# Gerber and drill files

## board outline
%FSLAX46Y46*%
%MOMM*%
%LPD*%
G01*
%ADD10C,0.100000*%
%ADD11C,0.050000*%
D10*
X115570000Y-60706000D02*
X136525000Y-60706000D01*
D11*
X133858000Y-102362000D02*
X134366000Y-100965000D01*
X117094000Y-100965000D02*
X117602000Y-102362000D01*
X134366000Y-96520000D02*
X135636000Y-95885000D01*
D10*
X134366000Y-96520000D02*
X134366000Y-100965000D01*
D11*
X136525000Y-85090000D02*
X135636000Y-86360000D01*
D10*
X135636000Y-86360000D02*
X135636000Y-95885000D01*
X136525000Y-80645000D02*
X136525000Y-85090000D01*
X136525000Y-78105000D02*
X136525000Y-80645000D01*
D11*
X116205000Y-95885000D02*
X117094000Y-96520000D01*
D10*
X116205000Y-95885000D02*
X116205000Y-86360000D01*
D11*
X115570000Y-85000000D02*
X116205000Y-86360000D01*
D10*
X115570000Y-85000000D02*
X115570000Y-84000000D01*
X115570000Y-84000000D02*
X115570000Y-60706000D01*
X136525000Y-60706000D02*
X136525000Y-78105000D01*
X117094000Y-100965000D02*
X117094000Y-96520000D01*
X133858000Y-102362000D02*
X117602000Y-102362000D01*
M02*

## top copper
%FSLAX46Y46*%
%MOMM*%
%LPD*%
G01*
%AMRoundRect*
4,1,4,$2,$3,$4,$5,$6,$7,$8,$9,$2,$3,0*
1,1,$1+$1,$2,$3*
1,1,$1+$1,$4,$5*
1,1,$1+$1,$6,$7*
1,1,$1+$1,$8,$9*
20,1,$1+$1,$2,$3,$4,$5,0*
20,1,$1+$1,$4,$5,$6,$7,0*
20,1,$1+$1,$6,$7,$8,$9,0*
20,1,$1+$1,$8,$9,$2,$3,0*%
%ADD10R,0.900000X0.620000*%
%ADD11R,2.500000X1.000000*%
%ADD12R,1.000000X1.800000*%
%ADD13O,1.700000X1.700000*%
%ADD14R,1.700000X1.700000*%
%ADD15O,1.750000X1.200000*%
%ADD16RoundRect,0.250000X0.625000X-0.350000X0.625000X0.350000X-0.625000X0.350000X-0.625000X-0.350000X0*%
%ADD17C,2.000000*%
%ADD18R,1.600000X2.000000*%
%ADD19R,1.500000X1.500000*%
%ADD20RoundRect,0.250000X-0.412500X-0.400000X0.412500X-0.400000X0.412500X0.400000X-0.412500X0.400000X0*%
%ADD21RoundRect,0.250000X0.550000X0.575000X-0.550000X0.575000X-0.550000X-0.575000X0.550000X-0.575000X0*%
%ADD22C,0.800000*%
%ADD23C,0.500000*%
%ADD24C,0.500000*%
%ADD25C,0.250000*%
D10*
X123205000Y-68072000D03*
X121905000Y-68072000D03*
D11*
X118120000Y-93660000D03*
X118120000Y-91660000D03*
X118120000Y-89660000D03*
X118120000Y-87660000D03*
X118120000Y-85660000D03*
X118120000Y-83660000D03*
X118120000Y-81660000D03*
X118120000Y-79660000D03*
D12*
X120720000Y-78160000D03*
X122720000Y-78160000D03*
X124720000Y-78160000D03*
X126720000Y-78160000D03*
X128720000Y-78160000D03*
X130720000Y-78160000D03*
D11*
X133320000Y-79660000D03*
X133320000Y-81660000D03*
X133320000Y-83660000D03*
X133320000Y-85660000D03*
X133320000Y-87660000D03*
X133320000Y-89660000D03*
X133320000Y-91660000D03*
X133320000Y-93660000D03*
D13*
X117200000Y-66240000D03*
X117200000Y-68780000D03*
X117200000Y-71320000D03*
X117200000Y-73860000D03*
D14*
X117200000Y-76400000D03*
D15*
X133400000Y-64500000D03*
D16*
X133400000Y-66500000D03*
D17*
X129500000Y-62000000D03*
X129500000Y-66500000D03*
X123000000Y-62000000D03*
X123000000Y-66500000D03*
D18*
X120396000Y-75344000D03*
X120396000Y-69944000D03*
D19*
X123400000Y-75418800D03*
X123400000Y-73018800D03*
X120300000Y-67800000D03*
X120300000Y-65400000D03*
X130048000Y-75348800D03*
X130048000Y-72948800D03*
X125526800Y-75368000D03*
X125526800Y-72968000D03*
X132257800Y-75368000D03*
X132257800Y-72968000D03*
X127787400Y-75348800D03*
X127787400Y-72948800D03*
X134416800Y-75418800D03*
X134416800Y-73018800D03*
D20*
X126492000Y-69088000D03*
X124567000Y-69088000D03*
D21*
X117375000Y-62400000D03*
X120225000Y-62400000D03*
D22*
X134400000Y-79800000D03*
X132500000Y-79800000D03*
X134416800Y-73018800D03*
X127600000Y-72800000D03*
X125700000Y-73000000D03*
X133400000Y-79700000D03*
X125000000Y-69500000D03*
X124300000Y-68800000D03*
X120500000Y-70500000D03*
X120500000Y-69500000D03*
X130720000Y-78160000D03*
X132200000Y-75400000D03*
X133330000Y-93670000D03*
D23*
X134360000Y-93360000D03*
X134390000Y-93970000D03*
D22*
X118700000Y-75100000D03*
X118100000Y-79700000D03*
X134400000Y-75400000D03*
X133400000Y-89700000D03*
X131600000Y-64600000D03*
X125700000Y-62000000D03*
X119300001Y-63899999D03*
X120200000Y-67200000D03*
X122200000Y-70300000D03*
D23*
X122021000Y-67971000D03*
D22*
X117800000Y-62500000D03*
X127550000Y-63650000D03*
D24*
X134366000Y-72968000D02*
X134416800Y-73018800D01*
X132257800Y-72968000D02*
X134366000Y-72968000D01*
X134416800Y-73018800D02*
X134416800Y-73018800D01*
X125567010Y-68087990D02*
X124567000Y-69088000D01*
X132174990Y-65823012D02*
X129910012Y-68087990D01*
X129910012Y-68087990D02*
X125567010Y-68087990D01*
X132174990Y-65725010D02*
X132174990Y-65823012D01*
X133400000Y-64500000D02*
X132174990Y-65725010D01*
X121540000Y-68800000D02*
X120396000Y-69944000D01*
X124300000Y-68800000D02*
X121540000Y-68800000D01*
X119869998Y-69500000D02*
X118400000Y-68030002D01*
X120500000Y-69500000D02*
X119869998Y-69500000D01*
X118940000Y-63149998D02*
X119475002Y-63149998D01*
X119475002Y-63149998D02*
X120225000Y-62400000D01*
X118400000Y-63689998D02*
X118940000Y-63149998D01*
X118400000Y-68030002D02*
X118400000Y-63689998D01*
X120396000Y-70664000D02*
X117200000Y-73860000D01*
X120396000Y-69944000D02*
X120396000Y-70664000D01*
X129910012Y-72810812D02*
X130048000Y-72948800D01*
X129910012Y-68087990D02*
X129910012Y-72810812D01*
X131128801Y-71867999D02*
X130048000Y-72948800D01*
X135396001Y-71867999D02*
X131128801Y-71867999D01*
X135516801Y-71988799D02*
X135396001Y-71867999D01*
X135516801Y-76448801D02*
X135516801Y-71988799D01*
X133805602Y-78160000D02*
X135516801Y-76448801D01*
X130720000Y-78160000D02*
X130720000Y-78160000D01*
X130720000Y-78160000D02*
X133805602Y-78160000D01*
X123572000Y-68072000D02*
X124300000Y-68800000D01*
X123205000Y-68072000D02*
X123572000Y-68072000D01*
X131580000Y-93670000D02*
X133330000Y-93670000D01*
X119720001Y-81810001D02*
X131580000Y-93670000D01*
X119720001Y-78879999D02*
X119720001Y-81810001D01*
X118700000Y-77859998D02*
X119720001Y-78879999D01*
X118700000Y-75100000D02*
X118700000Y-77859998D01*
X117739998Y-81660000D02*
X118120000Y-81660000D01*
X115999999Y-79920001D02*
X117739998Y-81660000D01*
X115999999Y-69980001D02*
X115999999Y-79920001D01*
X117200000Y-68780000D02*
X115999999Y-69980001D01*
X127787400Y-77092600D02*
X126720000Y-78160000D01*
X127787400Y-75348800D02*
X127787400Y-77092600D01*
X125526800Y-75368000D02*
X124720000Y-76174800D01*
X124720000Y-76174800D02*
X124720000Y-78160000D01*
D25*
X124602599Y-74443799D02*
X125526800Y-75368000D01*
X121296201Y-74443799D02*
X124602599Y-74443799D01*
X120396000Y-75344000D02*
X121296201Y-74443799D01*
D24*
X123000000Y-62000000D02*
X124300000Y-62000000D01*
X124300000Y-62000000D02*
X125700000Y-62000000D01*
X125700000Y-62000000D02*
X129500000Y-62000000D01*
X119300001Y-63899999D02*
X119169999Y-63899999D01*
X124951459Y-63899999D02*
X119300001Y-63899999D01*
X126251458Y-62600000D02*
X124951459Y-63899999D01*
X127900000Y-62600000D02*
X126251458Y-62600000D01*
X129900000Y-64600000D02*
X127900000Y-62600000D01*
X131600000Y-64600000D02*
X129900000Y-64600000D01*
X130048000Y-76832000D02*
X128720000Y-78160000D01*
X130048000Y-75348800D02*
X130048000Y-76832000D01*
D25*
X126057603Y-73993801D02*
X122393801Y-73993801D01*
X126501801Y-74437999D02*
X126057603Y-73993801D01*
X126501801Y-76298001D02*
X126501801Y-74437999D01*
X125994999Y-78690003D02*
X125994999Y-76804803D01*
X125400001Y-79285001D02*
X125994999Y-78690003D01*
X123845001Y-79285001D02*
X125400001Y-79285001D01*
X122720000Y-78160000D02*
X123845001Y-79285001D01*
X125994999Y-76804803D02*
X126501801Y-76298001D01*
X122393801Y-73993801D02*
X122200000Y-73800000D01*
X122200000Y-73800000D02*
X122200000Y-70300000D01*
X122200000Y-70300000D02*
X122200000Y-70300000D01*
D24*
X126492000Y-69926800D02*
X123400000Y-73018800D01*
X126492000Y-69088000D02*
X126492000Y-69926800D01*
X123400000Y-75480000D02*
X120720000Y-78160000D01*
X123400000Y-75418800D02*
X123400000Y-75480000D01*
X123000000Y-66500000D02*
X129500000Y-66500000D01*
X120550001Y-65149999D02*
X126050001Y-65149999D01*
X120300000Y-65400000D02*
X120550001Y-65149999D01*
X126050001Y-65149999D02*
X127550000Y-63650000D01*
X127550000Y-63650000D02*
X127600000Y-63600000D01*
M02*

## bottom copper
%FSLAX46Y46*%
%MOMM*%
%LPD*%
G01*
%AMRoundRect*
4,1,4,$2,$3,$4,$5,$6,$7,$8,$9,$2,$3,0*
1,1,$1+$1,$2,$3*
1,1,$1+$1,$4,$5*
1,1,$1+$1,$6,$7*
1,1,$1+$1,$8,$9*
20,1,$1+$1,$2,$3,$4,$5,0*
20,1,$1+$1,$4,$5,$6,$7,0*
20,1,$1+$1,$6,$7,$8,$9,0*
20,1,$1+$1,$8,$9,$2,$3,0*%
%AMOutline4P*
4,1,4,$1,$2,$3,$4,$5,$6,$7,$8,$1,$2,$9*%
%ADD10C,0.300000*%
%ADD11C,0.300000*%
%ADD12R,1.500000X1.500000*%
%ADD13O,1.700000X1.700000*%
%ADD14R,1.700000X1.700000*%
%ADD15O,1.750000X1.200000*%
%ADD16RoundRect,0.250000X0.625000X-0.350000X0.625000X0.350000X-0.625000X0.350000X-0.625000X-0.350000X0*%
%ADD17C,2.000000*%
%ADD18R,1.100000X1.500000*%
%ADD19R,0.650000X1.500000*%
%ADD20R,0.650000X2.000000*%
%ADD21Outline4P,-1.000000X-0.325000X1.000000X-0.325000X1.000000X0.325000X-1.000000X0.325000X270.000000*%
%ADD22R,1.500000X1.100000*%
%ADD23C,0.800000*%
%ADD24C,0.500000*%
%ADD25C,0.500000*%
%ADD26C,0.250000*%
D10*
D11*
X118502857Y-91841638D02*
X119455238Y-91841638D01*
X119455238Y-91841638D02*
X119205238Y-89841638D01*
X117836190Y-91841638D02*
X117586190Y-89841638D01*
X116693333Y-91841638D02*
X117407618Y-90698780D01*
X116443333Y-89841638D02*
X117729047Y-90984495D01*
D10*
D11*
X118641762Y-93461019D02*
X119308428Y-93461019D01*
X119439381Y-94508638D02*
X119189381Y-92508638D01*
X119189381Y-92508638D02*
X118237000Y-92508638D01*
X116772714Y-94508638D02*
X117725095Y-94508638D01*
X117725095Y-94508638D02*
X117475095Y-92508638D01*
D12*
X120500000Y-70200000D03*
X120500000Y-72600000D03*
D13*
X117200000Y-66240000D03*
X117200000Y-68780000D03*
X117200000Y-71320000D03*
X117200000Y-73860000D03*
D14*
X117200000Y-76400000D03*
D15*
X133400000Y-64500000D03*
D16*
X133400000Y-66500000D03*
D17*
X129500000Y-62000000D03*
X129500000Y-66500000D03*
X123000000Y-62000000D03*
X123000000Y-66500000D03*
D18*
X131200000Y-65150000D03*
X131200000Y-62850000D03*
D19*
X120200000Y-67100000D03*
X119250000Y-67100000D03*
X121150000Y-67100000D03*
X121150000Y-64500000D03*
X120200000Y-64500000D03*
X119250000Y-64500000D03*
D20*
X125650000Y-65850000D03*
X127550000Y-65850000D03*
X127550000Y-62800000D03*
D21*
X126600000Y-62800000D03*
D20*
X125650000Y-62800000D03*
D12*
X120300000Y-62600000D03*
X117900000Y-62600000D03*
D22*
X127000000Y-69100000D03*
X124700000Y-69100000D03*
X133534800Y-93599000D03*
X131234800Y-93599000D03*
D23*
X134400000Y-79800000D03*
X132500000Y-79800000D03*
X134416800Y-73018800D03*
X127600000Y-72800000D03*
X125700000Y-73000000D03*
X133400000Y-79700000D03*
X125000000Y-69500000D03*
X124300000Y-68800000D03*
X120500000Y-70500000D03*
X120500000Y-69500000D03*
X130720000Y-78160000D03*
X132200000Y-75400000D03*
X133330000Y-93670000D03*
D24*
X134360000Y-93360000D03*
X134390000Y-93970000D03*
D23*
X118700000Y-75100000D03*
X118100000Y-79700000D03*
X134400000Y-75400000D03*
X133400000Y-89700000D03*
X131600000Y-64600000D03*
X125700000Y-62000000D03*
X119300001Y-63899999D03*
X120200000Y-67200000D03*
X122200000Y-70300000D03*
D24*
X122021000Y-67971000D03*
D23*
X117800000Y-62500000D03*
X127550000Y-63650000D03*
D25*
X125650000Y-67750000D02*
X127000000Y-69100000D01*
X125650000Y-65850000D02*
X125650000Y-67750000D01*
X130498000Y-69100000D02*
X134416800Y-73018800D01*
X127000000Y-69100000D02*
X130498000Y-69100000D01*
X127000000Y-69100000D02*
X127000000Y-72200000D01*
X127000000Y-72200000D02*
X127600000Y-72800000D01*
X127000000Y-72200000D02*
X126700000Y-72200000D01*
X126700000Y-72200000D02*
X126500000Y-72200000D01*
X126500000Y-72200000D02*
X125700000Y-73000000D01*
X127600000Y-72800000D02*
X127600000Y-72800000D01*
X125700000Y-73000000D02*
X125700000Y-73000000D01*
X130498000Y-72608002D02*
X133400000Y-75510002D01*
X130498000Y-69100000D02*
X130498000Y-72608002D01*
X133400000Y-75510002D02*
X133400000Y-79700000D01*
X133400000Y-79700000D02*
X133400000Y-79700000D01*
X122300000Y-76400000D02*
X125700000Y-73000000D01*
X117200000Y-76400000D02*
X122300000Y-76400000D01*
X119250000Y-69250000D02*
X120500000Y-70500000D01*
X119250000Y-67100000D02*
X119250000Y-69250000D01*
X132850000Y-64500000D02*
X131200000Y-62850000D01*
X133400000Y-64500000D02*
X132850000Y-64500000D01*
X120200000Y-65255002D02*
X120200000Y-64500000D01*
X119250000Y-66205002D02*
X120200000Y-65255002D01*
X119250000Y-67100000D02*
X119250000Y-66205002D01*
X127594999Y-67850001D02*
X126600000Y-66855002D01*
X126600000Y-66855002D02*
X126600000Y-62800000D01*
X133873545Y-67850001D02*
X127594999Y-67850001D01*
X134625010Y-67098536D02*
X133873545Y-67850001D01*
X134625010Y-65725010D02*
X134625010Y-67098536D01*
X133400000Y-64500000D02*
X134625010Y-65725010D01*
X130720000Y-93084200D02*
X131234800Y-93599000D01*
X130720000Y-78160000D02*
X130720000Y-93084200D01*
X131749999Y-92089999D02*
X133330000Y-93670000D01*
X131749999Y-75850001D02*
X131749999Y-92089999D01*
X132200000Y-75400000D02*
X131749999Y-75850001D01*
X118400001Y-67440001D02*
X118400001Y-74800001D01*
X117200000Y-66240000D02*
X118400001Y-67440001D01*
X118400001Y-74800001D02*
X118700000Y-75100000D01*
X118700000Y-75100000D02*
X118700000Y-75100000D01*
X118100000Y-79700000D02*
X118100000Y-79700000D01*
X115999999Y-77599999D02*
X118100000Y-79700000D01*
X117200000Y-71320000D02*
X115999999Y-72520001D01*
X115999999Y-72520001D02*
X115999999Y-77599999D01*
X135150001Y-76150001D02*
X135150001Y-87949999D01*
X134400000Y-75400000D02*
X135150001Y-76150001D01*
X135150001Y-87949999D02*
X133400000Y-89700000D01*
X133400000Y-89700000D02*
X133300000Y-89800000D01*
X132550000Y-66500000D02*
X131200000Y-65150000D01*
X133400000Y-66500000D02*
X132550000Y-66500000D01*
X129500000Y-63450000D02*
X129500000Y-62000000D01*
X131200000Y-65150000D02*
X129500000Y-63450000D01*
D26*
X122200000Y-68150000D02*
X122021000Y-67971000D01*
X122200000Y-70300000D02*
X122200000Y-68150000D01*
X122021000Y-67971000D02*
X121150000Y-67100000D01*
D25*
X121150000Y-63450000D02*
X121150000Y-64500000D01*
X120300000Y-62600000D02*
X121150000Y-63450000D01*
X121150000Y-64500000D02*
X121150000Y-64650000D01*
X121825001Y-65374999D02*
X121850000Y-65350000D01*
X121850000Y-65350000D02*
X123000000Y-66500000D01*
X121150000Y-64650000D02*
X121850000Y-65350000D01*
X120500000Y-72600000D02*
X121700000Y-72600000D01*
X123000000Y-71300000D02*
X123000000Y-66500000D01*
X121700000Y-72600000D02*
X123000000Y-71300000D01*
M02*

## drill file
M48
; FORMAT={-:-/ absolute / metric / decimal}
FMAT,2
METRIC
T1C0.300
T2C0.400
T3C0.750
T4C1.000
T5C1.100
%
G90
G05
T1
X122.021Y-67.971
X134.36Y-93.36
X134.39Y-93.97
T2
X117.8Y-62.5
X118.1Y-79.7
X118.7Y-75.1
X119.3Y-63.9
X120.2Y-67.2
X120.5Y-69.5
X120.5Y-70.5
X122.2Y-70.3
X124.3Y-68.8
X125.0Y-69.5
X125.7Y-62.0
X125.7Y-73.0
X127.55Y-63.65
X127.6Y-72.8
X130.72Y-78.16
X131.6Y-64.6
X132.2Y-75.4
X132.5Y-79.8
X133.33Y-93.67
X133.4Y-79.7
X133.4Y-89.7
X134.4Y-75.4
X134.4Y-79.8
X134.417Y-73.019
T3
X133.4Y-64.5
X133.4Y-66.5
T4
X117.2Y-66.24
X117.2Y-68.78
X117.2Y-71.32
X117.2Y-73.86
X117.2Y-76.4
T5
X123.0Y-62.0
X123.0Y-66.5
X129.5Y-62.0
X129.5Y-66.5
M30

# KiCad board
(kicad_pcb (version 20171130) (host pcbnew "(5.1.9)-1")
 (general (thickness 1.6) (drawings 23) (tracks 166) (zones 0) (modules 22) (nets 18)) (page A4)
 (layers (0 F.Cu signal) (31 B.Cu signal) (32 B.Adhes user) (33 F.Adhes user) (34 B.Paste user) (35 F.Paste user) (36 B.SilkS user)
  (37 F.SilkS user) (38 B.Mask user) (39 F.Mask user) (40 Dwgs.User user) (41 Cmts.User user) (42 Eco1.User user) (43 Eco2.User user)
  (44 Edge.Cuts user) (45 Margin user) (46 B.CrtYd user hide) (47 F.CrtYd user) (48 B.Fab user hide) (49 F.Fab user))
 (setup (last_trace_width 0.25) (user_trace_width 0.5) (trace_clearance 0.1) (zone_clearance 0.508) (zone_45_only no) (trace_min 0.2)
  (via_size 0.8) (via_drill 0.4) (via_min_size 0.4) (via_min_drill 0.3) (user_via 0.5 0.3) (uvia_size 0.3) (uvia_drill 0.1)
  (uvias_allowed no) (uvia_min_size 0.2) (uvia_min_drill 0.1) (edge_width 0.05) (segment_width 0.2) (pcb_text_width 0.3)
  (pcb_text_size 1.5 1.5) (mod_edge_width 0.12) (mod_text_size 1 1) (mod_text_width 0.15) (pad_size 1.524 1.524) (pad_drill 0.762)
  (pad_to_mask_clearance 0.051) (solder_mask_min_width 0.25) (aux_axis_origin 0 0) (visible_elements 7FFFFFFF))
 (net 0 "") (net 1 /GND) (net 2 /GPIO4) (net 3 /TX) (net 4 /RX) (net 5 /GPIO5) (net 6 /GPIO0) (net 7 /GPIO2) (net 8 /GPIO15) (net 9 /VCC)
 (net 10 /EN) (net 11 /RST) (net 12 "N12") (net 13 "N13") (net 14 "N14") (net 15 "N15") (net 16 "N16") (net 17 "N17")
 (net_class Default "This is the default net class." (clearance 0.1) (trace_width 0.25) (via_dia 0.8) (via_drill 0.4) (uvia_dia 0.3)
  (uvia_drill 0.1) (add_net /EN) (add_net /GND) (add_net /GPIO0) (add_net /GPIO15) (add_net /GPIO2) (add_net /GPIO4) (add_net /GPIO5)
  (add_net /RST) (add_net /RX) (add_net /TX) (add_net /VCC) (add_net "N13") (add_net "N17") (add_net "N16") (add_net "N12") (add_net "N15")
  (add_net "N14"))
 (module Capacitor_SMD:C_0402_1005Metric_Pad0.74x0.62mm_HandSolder (layer F.Cu) (at 122.555 68.072)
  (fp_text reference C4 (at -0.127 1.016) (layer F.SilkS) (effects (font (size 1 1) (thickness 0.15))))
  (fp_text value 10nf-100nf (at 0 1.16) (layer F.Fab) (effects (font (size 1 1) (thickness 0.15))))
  (pad 2 smd rect (at 0.65 0) (size 0.9 0.62) (layers F.Cu F.Paste F.Mask) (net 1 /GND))
  (pad 1 smd rect (at -0.65 0) (size 0.9 0.62) (layers F.Cu F.Paste F.Mask) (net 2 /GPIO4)))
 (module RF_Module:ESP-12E (layer F.Cu) (at 125.72 90.16 180)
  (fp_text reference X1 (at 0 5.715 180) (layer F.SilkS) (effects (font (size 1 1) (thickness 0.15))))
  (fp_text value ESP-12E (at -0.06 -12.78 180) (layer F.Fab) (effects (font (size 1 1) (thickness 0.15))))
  (pad 22 smd rect (at 7.6 -3.5 180) (size 2.5 1) (layers F.Cu F.Paste F.Mask))
  (pad 21 smd rect (at 7.6 -1.5 180) (size 2.5 1) (layers F.Cu F.Paste F.Mask))
  (pad 20 smd rect (at 7.6 0.5 180) (size 2.5 1) (layers F.Cu F.Paste F.Mask))
  (pad 19 smd rect (at 7.6 2.5 180) (size 2.5 1) (layers F.Cu F.Paste F.Mask))
  (pad 18 smd rect (at 7.6 4.5 180) (size 2.5 1) (layers F.Cu F.Paste F.Mask))
  (pad 17 smd rect (at 7.6 6.5 180) (size 2.5 1) (layers F.Cu F.Paste F.Mask))
  (pad 16 smd rect (at 7.6 8.5 180) (size 2.5 1) (layers F.Cu F.Paste F.Mask) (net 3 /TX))
  (pad 15 smd rect (at 7.6 10.5 180) (size 2.5 1) (layers F.Cu F.Paste F.Mask) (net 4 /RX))
  (pad 14 smd rect (at 5 12 180) (size 1 1.8) (layers F.Cu F.Paste F.Mask) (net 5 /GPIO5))
  (pad 13 smd rect (at 3 12 180) (size 1 1.8) (layers F.Cu F.Paste F.Mask) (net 2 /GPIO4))
  (pad 12 smd rect (at 1 12 180) (size 1 1.8) (layers F.Cu F.Paste F.Mask) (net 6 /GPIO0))
  (pad 11 smd rect (at -1 12 180) (size 1 1.8) (layers F.Cu F.Paste F.Mask) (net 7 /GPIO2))
  (pad 10 smd rect (at -3 12 180) (size 1 1.8) (layers F.Cu F.Paste F.Mask) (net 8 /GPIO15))
  (pad 9 smd rect (at -5 12 180) (size 1 1.8) (layers F.Cu F.Paste F.Mask) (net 1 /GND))
  (pad 8 smd rect (at -7.6 10.5 180) (size 2.5 1) (layers F.Cu F.Paste F.Mask) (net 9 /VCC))
  (pad 7 smd rect (at -7.6 8.5 180) (size 2.5 1) (layers F.Cu F.Paste F.Mask))
  (pad 6 smd rect (at -7.6 6.5 180) (size 2.5 1) (layers F.Cu F.Paste F.Mask))
  (pad 5 smd rect (at -7.6 4.5 180) (size 2.5 1) (layers F.Cu F.Paste F.Mask))
  (pad 4 smd rect (at -7.6 2.5 180) (size 2.5 1) (layers F.Cu F.Paste F.Mask))
  (pad 3 smd rect (at -7.6 0.5 180) (size 2.5 1) (layers F.Cu F.Paste F.Mask) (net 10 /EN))
  (pad 2 smd rect (at -7.6 -1.5 180) (size 2.5 1) (layers F.Cu F.Paste F.Mask))
  (pad 1 smd rect (at -7.6 -3.5 180) (size 2.5 1) (layers F.Cu F.Paste F.Mask) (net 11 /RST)))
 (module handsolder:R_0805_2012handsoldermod (layer B.Cu) (at 120.5 71.4 90)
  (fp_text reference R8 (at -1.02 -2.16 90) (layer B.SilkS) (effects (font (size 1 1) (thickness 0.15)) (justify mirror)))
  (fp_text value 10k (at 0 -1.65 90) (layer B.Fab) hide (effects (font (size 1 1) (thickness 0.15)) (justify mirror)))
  (pad 2 smd rect (at 1.2 0 90) (size 1.5 1.5) (layers B.Cu B.Paste B.Mask) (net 1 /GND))
  (pad 1 smd rect (at -1.2 0 90) (size 1.5 1.5) (layers B.Cu B.Paste B.Mask) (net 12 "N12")))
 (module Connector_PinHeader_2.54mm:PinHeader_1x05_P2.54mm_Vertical (layer F.Cu) (at 117.2 76.4 180)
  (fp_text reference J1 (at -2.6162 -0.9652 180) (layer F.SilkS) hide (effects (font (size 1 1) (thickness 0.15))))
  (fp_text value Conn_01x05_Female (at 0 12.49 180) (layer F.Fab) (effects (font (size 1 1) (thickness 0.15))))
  (pad 5 thru_hole oval (at 0 10.16 180) (size 1.7 1.7) (drill 1) (layers *.Cu *.Mask) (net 11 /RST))
  (pad 4 thru_hole oval (at 0 7.62 180) (size 1.7 1.7) (drill 1) (layers *.Cu *.Mask) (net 3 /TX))
  (pad 3 thru_hole oval (at 0 5.08 180) (size 1.7 1.7) (drill 1) (layers *.Cu *.Mask) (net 4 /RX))
  (pad 2 thru_hole oval (at 0 2.54 180) (size 1.7 1.7) (drill 1) (layers *.Cu *.Mask) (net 1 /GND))
  (pad 1 thru_hole rect (at 0 0 180) (size 1.7 1.7) (drill 1) (layers *.Cu *.Mask) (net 9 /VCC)))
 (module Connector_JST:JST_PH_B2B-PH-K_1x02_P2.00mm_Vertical (layer F.Cu) (at 133.4 66.5 90)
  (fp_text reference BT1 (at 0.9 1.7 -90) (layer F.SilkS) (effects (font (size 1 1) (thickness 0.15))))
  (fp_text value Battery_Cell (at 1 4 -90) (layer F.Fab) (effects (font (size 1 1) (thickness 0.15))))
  (pad 2 thru_hole oval (at 2 0 90) (size 1.2 1.75) (drill 0.75) (layers *.Cu *.Mask) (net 1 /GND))
  (pad 1 thru_hole roundrect (at 0 0 90) (size 1.2 1.75) (drill 0.75) (layers *.Cu *.Mask) (roundrect_rratio 0.208333) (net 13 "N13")))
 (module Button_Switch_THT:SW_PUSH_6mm (layer F.Cu) (at 123 62)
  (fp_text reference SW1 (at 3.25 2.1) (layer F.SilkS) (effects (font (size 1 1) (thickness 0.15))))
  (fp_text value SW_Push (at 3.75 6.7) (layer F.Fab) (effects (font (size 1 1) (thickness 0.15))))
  (pad 1 thru_hole circle (at 6.5 0 90) (size 2 2) (drill 1.1) (layers *.Cu *.Mask) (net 13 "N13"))
  (pad 2 thru_hole circle (at 6.5 4.5 90) (size 2 2) (drill 1.1) (layers *.Cu *.Mask) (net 12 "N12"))
  (pad 1 thru_hole circle (at 0 0 90) (size 2 2) (drill 1.1) (layers *.Cu *.Mask) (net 13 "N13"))
  (pad 2 thru_hole circle (at 0 4.5 90) (size 2 2) (drill 1.1) (layers *.Cu *.Mask) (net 12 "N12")))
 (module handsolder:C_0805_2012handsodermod (layer B.Cu) (at 131.2 64 270)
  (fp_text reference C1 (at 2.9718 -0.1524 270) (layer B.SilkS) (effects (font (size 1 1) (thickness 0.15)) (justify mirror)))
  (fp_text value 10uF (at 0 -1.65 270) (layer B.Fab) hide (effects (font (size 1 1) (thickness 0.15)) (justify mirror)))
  (pad 2 smd rect (at 1.15 0 270) (size 1.5 1.1) (layers B.Cu B.Paste B.Mask) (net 13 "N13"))
  (pad 1 smd rect (at -1.15 0 270) (size 1.5 1.1) (layers B.Cu B.Paste B.Mask) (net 1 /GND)))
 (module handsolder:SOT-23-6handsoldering (layer B.Cu) (at 120.2 65.8 270)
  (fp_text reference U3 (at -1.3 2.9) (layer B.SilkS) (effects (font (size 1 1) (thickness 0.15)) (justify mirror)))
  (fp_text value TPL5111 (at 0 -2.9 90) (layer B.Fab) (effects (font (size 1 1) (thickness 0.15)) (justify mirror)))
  (pad 5 smd rect (at 1.3 0 270) (size 1.5 0.65) (layers B.Cu B.Paste B.Mask) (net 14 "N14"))
  (pad 6 smd rect (at 1.3 0.95 270) (size 1.5 0.65) (layers B.Cu B.Paste B.Mask) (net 1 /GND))
  (pad 4 smd rect (at 1.3 -0.95 270) (size 1.5 0.65) (layers B.Cu B.Paste B.Mask) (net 2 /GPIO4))
  (pad 3 smd rect (at -1.3 -0.95 270) (size 1.5 0.65) (layers B.Cu B.Paste B.Mask) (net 12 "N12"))
  (pad 2 smd rect (at -1.3 0 270) (size 1.5 0.65) (layers B.Cu B.Paste B.Mask) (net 1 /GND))
  (pad 1 smd rect (at -1.3 0.95 270) (size 1.5 0.65) (layers B.Cu B.Paste B.Mask) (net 13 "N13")))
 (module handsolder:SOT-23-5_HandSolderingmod (layer B.Cu) (at 126.6 64.35 270)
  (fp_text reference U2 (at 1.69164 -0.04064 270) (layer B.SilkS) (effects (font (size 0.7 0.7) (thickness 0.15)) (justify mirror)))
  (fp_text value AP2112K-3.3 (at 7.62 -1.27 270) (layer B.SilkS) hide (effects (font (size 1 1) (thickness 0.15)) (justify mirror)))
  (pad 5 smd rect (at 1.5 0.95 270) (size 2 0.65) (layers B.Cu B.Paste B.Mask) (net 9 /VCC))
  (pad 4 smd rect (at 1.5 -0.95 270) (size 2 0.65) (layers B.Cu B.Paste B.Mask))
  (pad 3 smd rect (at -1.55 -0.95 270) (size 2 0.65) (layers B.Cu B.Paste B.Mask) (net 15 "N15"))
  (pad 2 smd trapezoid (at -1.55 0 270) (size 2 0.65) (layers B.Cu B.Paste B.Mask) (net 1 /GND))
  (pad 1 smd rect (at -1.55 0.95 270) (size 2 0.65) (layers B.Cu B.Paste B.Mask) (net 13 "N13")))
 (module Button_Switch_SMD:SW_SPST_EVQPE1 (layer F.Cu) (at 120.396 72.644 90)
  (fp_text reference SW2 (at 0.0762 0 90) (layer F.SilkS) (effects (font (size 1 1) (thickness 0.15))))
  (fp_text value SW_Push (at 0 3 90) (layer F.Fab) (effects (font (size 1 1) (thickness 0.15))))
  (pad 1 smd rect (at -2.7 0 90) (size 2 1.6) (layers F.Cu F.Paste F.Mask) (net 6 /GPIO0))
  (pad 2 smd rect (at 2.7 0 90) (size 2 1.6) (layers F.Cu F.Paste F.Mask) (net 1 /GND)))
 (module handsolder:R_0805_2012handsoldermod (layer F.Cu) (at 123.4 74.2188 270)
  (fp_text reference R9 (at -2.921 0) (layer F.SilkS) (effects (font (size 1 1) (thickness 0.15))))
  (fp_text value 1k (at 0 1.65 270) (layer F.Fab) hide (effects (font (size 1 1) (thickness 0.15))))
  (pad 2 smd rect (at 1.2 0 270) (size 1.5 1.5) (layers F.Cu F.Paste F.Mask) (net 5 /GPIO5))
  (pad 1 smd rect (at -1.2 0 270) (size 1.5 1.5) (layers F.Cu F.Paste F.Mask) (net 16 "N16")))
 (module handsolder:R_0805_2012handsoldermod (layer F.Cu) (at 120.3 66.6 270)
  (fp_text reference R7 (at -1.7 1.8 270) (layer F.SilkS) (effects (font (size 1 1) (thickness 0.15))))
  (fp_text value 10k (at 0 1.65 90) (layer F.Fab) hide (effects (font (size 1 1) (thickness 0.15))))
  (pad 2 smd rect (at 1.2 0 270) (size 1.5 1.5) (layers F.Cu F.Paste F.Mask) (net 14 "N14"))
  (pad 1 smd rect (at -1.2 0 270) (size 1.5 1.5) (layers F.Cu F.Paste F.Mask) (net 15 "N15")))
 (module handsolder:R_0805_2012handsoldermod (layer B.Cu) (at 119.1 62.6)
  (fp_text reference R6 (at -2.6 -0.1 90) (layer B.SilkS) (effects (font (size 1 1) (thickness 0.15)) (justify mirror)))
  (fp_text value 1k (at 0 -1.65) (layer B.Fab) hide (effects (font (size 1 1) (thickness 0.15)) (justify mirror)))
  (pad 2 smd rect (at 1.2 0) (size 1.5 1.5) (layers B.Cu B.Paste B.Mask) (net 12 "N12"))
  (pad 1 smd rect (at -1.2 0) (size 1.5 1.5) (layers B.Cu B.Paste B.Mask) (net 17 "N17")))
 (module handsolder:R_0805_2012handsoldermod (layer F.Cu) (at 130.048 74.1488 270)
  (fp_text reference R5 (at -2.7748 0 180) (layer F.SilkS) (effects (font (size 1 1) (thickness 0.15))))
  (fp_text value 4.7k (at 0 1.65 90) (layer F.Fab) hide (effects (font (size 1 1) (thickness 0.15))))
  (pad 2 smd rect (at 1.2 0 270) (size 1.5 1.5) (layers F.Cu F.Paste F.Mask) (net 8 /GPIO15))
  (pad 1 smd rect (at -1.2 0 270) (size 1.5 1.5) (layers F.Cu F.Paste F.Mask) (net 1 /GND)))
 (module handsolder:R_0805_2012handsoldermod (layer F.Cu) (at 125.5268 74.168 270)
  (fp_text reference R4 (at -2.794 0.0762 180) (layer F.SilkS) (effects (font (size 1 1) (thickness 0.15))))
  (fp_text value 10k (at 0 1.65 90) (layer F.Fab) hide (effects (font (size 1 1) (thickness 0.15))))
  (pad 2 smd rect (at 1.2 0 270) (size 1.5 1.5) (layers F.Cu F.Paste F.Mask) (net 6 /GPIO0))
  (pad 1 smd rect (at -1.2 0 270) (size 1.5 1.5) (layers F.Cu F.Paste F.Mask) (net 9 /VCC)))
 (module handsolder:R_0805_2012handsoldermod (layer F.Cu) (at 132.2578 74.168 270)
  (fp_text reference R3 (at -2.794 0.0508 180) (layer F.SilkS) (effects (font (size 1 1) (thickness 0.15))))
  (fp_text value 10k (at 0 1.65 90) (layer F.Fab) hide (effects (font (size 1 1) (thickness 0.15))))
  (pad 2 smd rect (at 1.2 0 270) (size 1.5 1.5) (layers F.Cu F.Paste F.Mask) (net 11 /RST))
  (pad 1 smd rect (at -1.2 0 270) (size 1.5 1.5) (layers F.Cu F.Paste F.Mask) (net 9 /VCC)))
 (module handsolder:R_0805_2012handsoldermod (layer F.Cu) (at 127.7874 74.1488 270)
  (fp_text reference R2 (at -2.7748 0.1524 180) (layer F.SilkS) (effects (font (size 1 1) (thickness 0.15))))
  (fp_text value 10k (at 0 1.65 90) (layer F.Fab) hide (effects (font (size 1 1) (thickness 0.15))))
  (pad 2 smd rect (at 1.2 0 270) (size 1.5 1.5) (layers F.Cu F.Paste F.Mask) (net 7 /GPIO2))
  (pad 1 smd rect (at -1.2 0 270) (size 1.5 1.5) (layers F.Cu F.Paste F.Mask) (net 9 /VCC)))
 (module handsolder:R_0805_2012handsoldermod (layer F.Cu) (at 134.4168 74.2188 270)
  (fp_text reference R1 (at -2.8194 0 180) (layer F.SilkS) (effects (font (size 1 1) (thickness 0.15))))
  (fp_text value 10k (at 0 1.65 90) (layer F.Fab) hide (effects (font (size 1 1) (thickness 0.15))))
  (pad 2 smd rect (at 1.2 0 270) (size 1.5 1.5) (layers F.Cu F.Paste F.Mask) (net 10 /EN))
  (pad 1 smd rect (at -1.2 0 270) (size 1.5 1.5) (layers F.Cu F.Paste F.Mask) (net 9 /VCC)))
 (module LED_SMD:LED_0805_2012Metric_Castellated (layer F.Cu) (at 125.5295 69.088)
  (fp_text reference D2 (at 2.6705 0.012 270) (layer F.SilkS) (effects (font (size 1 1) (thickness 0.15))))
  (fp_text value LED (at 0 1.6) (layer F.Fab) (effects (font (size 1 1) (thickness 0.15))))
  (pad 2 smd roundrect (at 0.9625 0) (size 1.325 1.3) (layers F.Cu F.Paste F.Mask) (roundrect_rratio 0.1923076923076923) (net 16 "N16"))
  (pad 1 smd roundrect (at -0.9625 0) (size 1.325 1.3) (layers F.Cu F.Paste F.Mask) (roundrect_rratio 0.1923076923076923) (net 1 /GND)))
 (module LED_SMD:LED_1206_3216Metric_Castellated (layer F.Cu) (at 118.8 62.4 180)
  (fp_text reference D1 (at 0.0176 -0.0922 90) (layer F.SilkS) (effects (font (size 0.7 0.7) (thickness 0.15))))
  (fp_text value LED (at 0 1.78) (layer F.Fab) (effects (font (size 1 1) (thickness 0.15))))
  (pad 2 smd roundrect (at 1.425 0 180) (size 1.6 1.65) (layers F.Cu F.Paste F.Mask) (roundrect_rratio 0.15625) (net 17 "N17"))
  (pad 1 smd roundrect (at -1.425 0 180) (size 1.6 1.65) (layers F.Cu F.Paste F.Mask) (roundrect_rratio 0.15625) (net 1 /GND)))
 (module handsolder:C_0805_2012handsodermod (layer B.Cu) (at 125.85 69.1)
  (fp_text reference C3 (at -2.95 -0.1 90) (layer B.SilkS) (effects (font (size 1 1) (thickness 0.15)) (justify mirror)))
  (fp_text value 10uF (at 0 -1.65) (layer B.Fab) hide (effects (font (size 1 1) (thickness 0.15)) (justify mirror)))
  (pad 2 smd rect (at 1.15 0) (size 1.5 1.1) (layers B.Cu B.Paste B.Mask) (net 9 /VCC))
  (pad 1 smd rect (at -1.15 0) (size 1.5 1.1) (layers B.Cu B.Paste B.Mask) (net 1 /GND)))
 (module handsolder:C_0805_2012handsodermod (layer B.Cu) (at 132.3848 93.599)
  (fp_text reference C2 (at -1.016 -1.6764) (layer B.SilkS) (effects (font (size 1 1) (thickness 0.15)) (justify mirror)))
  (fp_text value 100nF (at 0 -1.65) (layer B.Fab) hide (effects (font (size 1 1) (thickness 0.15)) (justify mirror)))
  (pad 2 smd rect (at 1.15 0) (size 1.5 1.1) (layers B.Cu B.Paste B.Mask) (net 11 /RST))
  (pad 1 smd rect (at -1.15 0) (size 1.5 1.1) (layers B.Cu B.Paste B.Mask) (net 1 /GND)))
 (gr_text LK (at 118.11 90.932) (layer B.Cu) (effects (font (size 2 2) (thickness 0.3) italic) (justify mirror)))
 (gr_line (start 115.57 60.706) (end 136.525 60.706) (layer Edge.Cuts) (width 0.1))
 (gr_line (start 133.858 102.362) (end 134.366 100.965) (layer Edge.Cuts) (width 0.05))
 (gr_line (start 117.094 100.965) (end 117.602 102.362) (layer Edge.Cuts) (width 0.05))
 (gr_line (start 134.366 96.52) (end 135.636 95.885) (layer Edge.Cuts) (width 0.05))
 (gr_line (start 134.366 96.52) (end 134.366 100.965) (layer Edge.Cuts) (width 0.1))
 (gr_line (start 136.525 85.09) (end 135.636 86.36) (layer Edge.Cuts) (width 0.05))
 (gr_line (start 135.636 86.36) (end 135.636 95.885) (layer Edge.Cuts) (width 0.1))
 (gr_line (start 136.525 80.645) (end 136.525 85.09) (layer Edge.Cuts) (width 0.1))
 (gr_line (start 136.525 78.105) (end 136.525 80.645) (layer Edge.Cuts) (width 0.1))
 (gr_line (start 116.205 95.885) (end 117.094 96.52) (layer Edge.Cuts) (width 0.05))
 (gr_line (start 116.205 95.885) (end 116.205 86.36) (layer Edge.Cuts) (width 0.1))
 (gr_line (start 115.57 85) (end 116.205 86.36) (layer Edge.Cuts) (width 0.05))
 (gr_line (start 115.57 85) (end 115.57 84) (layer Edge.Cuts) (width 0.1))
 (gr_line (start 115.57 84) (end 115.57 60.706) (layer Edge.Cuts) (width 0.1))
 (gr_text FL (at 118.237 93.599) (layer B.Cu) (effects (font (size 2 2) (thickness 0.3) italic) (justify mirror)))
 (gr_line (start 136.525 60.706) (end 136.525 78.105) (layer Edge.Cuts) (width 0.1))
 (gr_line (start 117.094 100.965) (end 117.094 96.52) (layer Edge.Cuts) (width 0.1))
 (gr_line (start 133.858 102.362) (end 117.602 102.362) (layer Edge.Cuts) (width 0.1))
 (via (at 134.4 79.8) (size 0.8) (drill 0.4) (layers F.Cu B.Cu) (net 9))
 (via (at 132.5 79.8) (size 0.8) (drill 0.4) (layers F.Cu B.Cu) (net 9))
 (segment (start 125.65 67.75) (end 127 69.1) (width 0.5) (layer B.Cu) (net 9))
 (segment (start 125.65 65.85) (end 125.65 67.75) (width 0.5) (layer B.Cu) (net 9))
 (segment (start 134.366 72.968) (end 134.4168 73.0188) (width 0.5) (layer F.Cu) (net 9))
 (segment (start 132.2578 72.968) (end 134.366 72.968) (width 0.5) (layer F.Cu) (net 9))
 (segment (start 134.4168 73.0188) (end 134.4168 73.0188) (width 0.5) (layer F.Cu) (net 9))
 (via (at 134.4168 73.0188) (size 0.8) (drill 0.4) (layers F.Cu B.Cu) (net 9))
 (segment (start 130.498 69.1) (end 134.4168 73.0188) (width 0.5) (layer B.Cu) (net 9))
 (segment (start 127 69.1) (end 130.498 69.1) (width 0.5) (layer B.Cu) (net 9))
 (segment (start 127 69.1) (end 127 72.2) (width 0.5) (layer B.Cu) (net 9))
 (segment (start 127 72.2) (end 127.6 72.8) (width 0.5) (layer B.Cu) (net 9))
 (segment (start 127 72.2) (end 126.7 72.2) (width 0.5) (layer B.Cu) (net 9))
 (segment (start 126.7 72.2) (end 126.5 72.2) (width 0.5) (layer B.Cu) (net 9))
 (segment (start 126.5 72.2) (end 125.7 73) (width 0.5) (layer B.Cu) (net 9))
 (segment (start 127.6 72.8) (end 127.6 72.8) (width 0.5) (layer B.Cu) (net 9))
 (via (at 127.6 72.8) (size 0.8) (drill 0.4) (layers F.Cu B.Cu) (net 9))
 (segment (start 125.7 73) (end 125.7 73) (width 0.5) (layer B.Cu) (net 9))
 (via (at 125.7 73) (size 0.8) (drill 0.4) (layers F.Cu B.Cu) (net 9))
 (segment (start 130.498 72.608002) (end 133.4 75.510002) (width 0.5) (layer B.Cu) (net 9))
 (segment (start 130.498 69.1) (end 130.498 72.608002) (width 0.5) (layer B.Cu) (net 9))
 (segment (start 133.4 75.510002) (end 133.4 79.7) (width 0.5) (layer B.Cu) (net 9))
 (segment (start 133.4 79.7) (end 133.4 79.7) (width 0.5) (layer B.Cu) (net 9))
 (via (at 133.4 79.7) (size 0.8) (drill 0.4) (layers F.Cu B.Cu) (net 9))
 (segment (start 122.3 76.4) (end 125.7 73) (width 0.5) (layer B.Cu) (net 9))
 (segment (start 117.2 76.4) (end 122.3 76.4) (width 0.5) (layer B.Cu) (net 9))
 (via (at 125 69.5) (size 0.8) (drill 0.4) (layers F.Cu B.Cu) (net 1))
 (via (at 124.3 68.8) (size 0.8) (drill 0.4) (layers F.Cu B.Cu) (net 1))
 (via (at 120.5 70.5) (size 0.8) (drill 0.4) (layers F.Cu B.Cu) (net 1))
 (via (at 120.5 69.5) (size 0.8) (drill 0.4) (layers F.Cu B.Cu) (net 1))
 (segment (start 119.25 69.25) (end 120.5 70.5) (width 0.5) (layer B.Cu) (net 1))
 (segment (start 119.25 67.1) (end 119.25 69.25) (width 0.5) (layer B.Cu) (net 1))
 (segment (start 132.85 64.5) (end 131.2 62.85) (width 0.5) (layer B.Cu) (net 1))
 (segment (start 133.4 64.5) (end 132.85 64.5) (width 0.5) (layer B.Cu) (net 1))
 (segment (start 120.2 65.255002) (end 120.2 64.5) (width 0.5) (layer B.Cu) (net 1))
 (segment (start 119.25 66.205002) (end 120.2 65.255002) (width 0.5) (layer B.Cu) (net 1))
 (segment (start 119.25 67.1) (end 119.25 66.205002) (width 0.5) (layer B.Cu) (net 1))
 (segment (start 127.594999 67.850001) (end 126.6 66.855002) (width 0.5) (layer B.Cu) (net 1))
 (segment (start 126.6 66.855002) (end 126.6 62.8) (width 0.5) (layer B.Cu) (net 1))
 (segment (start 133.873545 67.850001) (end 127.594999 67.850001) (width 0.5) (layer B.Cu) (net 1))
 (segment (start 134.62501 67.098536) (end 133.873545 67.850001) (width 0.5) (layer B.Cu) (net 1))
 (segment (start 134.62501 65.72501) (end 134.62501 67.098536) (width 0.5) (layer B.Cu) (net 1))
 (segment (start 133.4 64.5) (end 134.62501 65.72501) (width 0.5) (layer B.Cu) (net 1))
 (segment (start 125.56701 68.08799) (end 124.567 69.088) (width 0.5) (layer F.Cu) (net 1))
 (segment (start 132.17499 65.823012) (end 129.910012 68.08799) (width 0.5) (layer F.Cu) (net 1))
 (segment (start 129.910012 68.08799) (end 125.56701 68.08799) (width 0.5) (layer F.Cu) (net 1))
 (segment (start 132.17499 65.72501) (end 132.17499 65.823012) (width 0.5) (layer F.Cu) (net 1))
 (segment (start 133.4 64.5) (end 132.17499 65.72501) (width 0.5) (layer F.Cu) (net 1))
 (segment (start 121.54 68.8) (end 120.396 69.944) (width 0.5) (layer F.Cu) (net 1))
 (segment (start 124.3 68.8) (end 121.54 68.8) (width 0.5) (layer F.Cu) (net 1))
 (segment (start 119.869998 69.5) (end 118.4 68.030002) (width 0.5) (layer F.Cu) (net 1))
 (segment (start 120.5 69.5) (end 119.869998 69.5) (width 0.5) (layer F.Cu) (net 1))
 (segment (start 118.94 63.149998) (end 119.475002 63.149998) (width 0.5) (layer F.Cu) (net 1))
 (segment (start 119.475002 63.149998) (end 120.225 62.4) (width 0.5) (layer F.Cu) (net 1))
 (segment (start 118.4 63.689998) (end 118.94 63.149998) (width 0.5) (layer F.Cu) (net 1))
 (segment (start 118.4 68.030002) (end 118.4 63.689998) (width 0.5) (layer F.Cu) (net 1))
 (segment (start 120.396 70.664) (end 117.2 73.86) (width 0.5) (layer F.Cu) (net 1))
 (segment (start 120.396 69.944) (end 120.396 70.664) (width 0.5) (layer F.Cu) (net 1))
 (segment (start 129.910012 72.810812) (end 130.048 72.9488) (width 0.5) (layer F.Cu) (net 1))
 (segment (start 129.910012 68.08799) (end 129.910012 72.810812) (width 0.5) (layer F.Cu) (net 1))
 (segment (start 131.128801 71.867999) (end 130.048 72.9488) (width 0.5) (layer F.Cu) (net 1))
 (segment (start 135.396001 71.867999) (end 131.128801 71.867999) (width 0.5) (layer F.Cu) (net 1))
 (segment (start 135.516801 71.988799) (end 135.396001 71.867999) (width 0.5) (layer F.Cu) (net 1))
 (segment (start 135.516801 76.448801) (end 135.516801 71.988799) (width 0.5) (layer F.Cu) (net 1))
 (segment (start 133.805602 78.16) (end 135.516801 76.448801) (width 0.5) (layer F.Cu) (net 1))
 (segment (start 130.72 78.16) (end 130.72 78.16) (width 0.5) (layer F.Cu) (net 1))
 (segment (start 130.72 78.16) (end 133.805602 78.16) (width 0.5) (layer F.Cu) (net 1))
 (via (at 130.72 78.16) (size 0.8) (drill 0.4) (layers F.Cu B.Cu) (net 1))
 (segment (start 130.72 93.0842) (end 131.2348 93.599) (width 0.5) (layer B.Cu) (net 1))
 (segment (start 130.72 78.16) (end 130.72 93.0842) (width 0.5) (layer B.Cu) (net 1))
 (segment (start 123.572 68.072) (end 124.3 68.8) (width 0.5) (layer F.Cu) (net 1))
 (segment (start 123.205 68.072) (end 123.572 68.072) (width 0.5) (layer F.Cu) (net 1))
 (via (at 132.2 75.4) (size 0.8) (drill 0.4) (layers F.Cu B.Cu) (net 11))
 (via (at 133.33 93.67) (size 0.8) (drill 0.4) (layers F.Cu B.Cu) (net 11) (status 30))
 (via (at 134.36 93.36) (size 0.5) (drill 0.3) (layers F.Cu B.Cu) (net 11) (status 30))
 (via (at 134.39 93.97) (size 0.5) (drill 0.3) (layers F.Cu B.Cu) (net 11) (status 30))
 (segment (start 131.749999 92.089999) (end 133.33 93.67) (width 0.5) (layer B.Cu) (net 11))
 (segment (start 131.749999 75.850001) (end 131.749999 92.089999) (width 0.5) (layer B.Cu) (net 11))
 (segment (start 132.2 75.4) (end 131.749999 75.850001) (width 0.5) (layer B.Cu) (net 11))
 (segment (start 118.400001 67.440001) (end 118.400001 74.800001) (width 0.5) (layer B.Cu) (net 11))
 (segment (start 117.2 66.24) (end 118.400001 67.440001) (width 0.5) (layer B.Cu) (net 11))
 (segment (start 118.400001 74.800001) (end 118.7 75.1) (width 0.5) (layer B.Cu) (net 11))
 (segment (start 118.7 75.1) (end 118.7 75.1) (width 0.5) (layer B.Cu) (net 11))
 (via (at 118.7 75.1) (size 0.8) (drill 0.4) (layers F.Cu B.Cu) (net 11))
 (segment (start 131.58 93.67) (end 133.33 93.67) (width 0.5) (layer F.Cu) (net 11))
 (segment (start 119.720001 81.810001) (end 131.58 93.67) (width 0.5) (layer F.Cu) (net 11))
 (segment (start 119.720001 78.879999) (end 119.720001 81.810001) (width 0.5) (layer F.Cu) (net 11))
 (segment (start 118.7 77.859998) (end 119.720001 78.879999) (width 0.5) (layer F.Cu) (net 11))
 (segment (start 118.7 75.1) (end 118.7 77.859998) (width 0.5) (layer F.Cu) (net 11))
 (segment (start 118.1 79.7) (end 118.1 79.7) (width 0.5) (layer B.Cu) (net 4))
 (via (at 118.1 79.7) (size 0.8) (drill 0.4) (layers F.Cu B.Cu) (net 4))
 (segment (start 115.999999 77.599999) (end 118.1 79.7) (width 0.5) (layer B.Cu) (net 4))
 (segment (start 117.2 71.32) (end 115.999999 72.520001) (width 0.5) (layer B.Cu) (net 4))
 (segment (start 115.999999 72.520001) (end 115.999999 77.599999) (width 0.5) (layer B.Cu) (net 4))
 (segment (start 117.739998 81.66) (end 118.12 81.66) (width 0.5) (layer F.Cu) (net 3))
 (segment (start 115.999999 79.920001) (end 117.739998 81.66) (width 0.5) (layer F.Cu) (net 3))
 (segment (start 115.999999 69.980001) (end 115.999999 79.920001) (width 0.5) (layer F.Cu) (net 3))
 (segment (start 117.2 68.78) (end 115.999999 69.980001) (width 0.5) (layer F.Cu) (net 3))
 (via (at 134.4 75.4) (size 0.8) (drill 0.4) (layers F.Cu B.Cu) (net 10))
 (segment (start 135.150001 76.150001) (end 135.150001 87.949999) (width 0.5) (layer B.Cu) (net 10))
 (segment (start 134.4 75.4) (end 135.150001 76.150001) (width 0.5) (layer B.Cu) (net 10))
 (segment (start 135.150001 87.949999) (end 133.4 89.7) (width 0.5) (layer B.Cu) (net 10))
 (segment (start 133.4 89.7) (end 133.3 89.8) (width 0.5) (layer B.Cu) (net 10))
 (via (at 133.4 89.7) (size 0.8) (drill 0.4) (layers F.Cu B.Cu) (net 10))
 (segment (start 127.7874 77.0926) (end 126.72 78.16) (width 0.5) (layer F.Cu) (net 7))
 (segment (start 127.7874 75.3488) (end 127.7874 77.0926) (width 0.5) (layer F.Cu) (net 7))
 (segment (start 125.5268 75.368) (end 124.72 76.1748) (width 0.5) (layer F.Cu) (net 6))
 (segment (start 124.72 76.1748) (end 124.72 78.16) (width 0.5) (layer F.Cu) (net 6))
 (segment (start 124.602599 74.443799) (end 125.5268 75.368) (width 0.25) (layer F.Cu) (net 6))
 (segment (start 121.296201 74.443799) (end 124.602599 74.443799) (width 0.25) (layer F.Cu) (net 6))
 (segment (start 120.396 75.344) (end 121.296201 74.443799) (width 0.25) (layer F.Cu) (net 6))
 (via (at 131.6 64.6) (size 0.8) (drill 0.4) (layers F.Cu B.Cu) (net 13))
 (segment (start 123 62) (end 124.3 62) (width 0.5) (layer F.Cu) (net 13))
 (segment (start 124.3 62) (end 125.7 62) (width 0.5) (layer F.Cu) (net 13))
 (segment (start 125.7 62) (end 129.5 62) (width 0.5) (layer F.Cu) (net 13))
 (via (at 125.7 62) (size 0.8) (drill 0.4) (layers F.Cu B.Cu) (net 13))
 (segment (start 132.55 66.5) (end 131.2 65.15) (width 0.5) (layer B.Cu) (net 13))
 (segment (start 133.4 66.5) (end 132.55 66.5) (width 0.5) (layer B.Cu) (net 13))
 (segment (start 129.5 63.45) (end 129.5 62) (width 0.5) (layer B.Cu) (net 13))
 (segment (start 131.2 65.15) (end 129.5 63.45) (width 0.5) (layer B.Cu) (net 13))
 (segment (start 119.300001 63.899999) (end 119.169999 63.899999) (width 0.5) (layer F.Cu) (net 13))
 (via (at 119.300001 63.899999) (size 0.8) (drill 0.4) (layers F.Cu B.Cu) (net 13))
 (segment (start 124.951459 63.899999) (end 119.300001 63.899999) (width 0.5) (layer F.Cu) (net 13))
 (segment (start 126.251458 62.6) (end 124.951459 63.899999) (width 0.5) (layer F.Cu) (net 13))
 (segment (start 127.9 62.6) (end 126.251458 62.6) (width 0.5) (layer F.Cu) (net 13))
 (segment (start 129.9 64.6) (end 127.9 62.6) (width 0.5) (layer F.Cu) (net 13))
 (segment (start 131.6 64.6) (end 129.9 64.6) (width 0.5) (layer F.Cu) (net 13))
 (segment (start 130.048 76.832) (end 128.72 78.16) (width 0.5) (layer F.Cu) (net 8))
 (segment (start 130.048 75.3488) (end 130.048 76.832) (width 0.5) (layer F.Cu) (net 8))
 (via (at 120.2 67.2) (size 0.8) (drill 0.4) (layers F.Cu B.Cu) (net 14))
 (segment (start 126.057603 73.993801) (end 122.393801 73.993801) (width 0.25) (layer F.Cu) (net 2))
 (segment (start 126.501801 74.437999) (end 126.057603 73.993801) (width 0.25) (layer F.Cu) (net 2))
 (segment (start 126.501801 76.298001) (end 126.501801 74.437999) (width 0.25) (layer F.Cu) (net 2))
 (segment (start 125.994999 78.690003) (end 125.994999 76.804803) (width 0.25) (layer F.Cu) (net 2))
 (segment (start 125.400001 79.285001) (end 125.994999 78.690003) (width 0.25) (layer F.Cu) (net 2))
 (segment (start 123.845001 79.285001) (end 125.400001 79.285001) (width 0.25) (layer F.Cu) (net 2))
 (segment (start 122.72 78.16) (end 123.845001 79.285001) (width 0.25) (layer F.Cu) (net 2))
 (segment (start 125.994999 76.804803) (end 126.501801 76.298001) (width 0.25) (layer F.Cu) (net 2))
 (segment (start 122.393801 73.993801) (end 122.2 73.8) (width 0.25) (layer F.Cu) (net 2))
 (segment (start 122.2 73.8) (end 122.2 70.3) (width 0.25) (layer F.Cu) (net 2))
 (segment (start 122.2 70.3) (end 122.2 70.3) (width 0.25) (layer F.Cu) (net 2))
 (via (at 122.2 70.3) (size 0.8) (drill 0.4) (layers F.Cu B.Cu) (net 2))
 (segment (start 122.2 68.15) (end 122.021 67.971) (width 0.25) (layer B.Cu) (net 2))
 (segment (start 122.2 70.3) (end 122.2 68.15) (width 0.25) (layer B.Cu) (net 2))
 (segment (start 122.021 67.971) (end 121.15 67.1) (width 0.25) (layer B.Cu) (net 2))
 (via (at 122.021 67.971) (size 0.5) (drill 0.3) (layers F.Cu B.Cu) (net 2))
 (segment (start 126.492 69.9268) (end 123.4 73.0188) (width 0.5) (layer F.Cu) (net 16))
 (segment (start 126.492 69.088) (end 126.492 69.9268) (width 0.5) (layer F.Cu) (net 16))
 (segment (start 123.4 75.48) (end 120.72 78.16) (width 0.5) (layer F.Cu) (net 5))
 (segment (start 123.4 75.4188) (end 123.4 75.48) (width 0.5) (layer F.Cu) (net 5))
 (via (at 117.8 62.5) (size 0.8) (drill 0.4) (layers F.Cu B.Cu) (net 17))
 (segment (start 121.15 63.45) (end 121.15 64.5) (width 0.5) (layer B.Cu) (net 12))
 (segment (start 120.3 62.6) (end 121.15 63.45) (width 0.5) (layer B.Cu) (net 12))
 (segment (start 121.15 64.5) (end 121.15 64.65) (width 0.5) (layer B.Cu) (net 12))
 (segment (start 121.825001 65.374999) (end 121.85 65.35) (width 0.5) (layer B.Cu) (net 12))
 (segment (start 121.85 65.35) (end 123 66.5) (width 0.5) (layer B.Cu) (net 12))
 (segment (start 121.15 64.65) (end 121.85 65.35) (width 0.5) (layer B.Cu) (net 12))
 (segment (start 123 66.5) (end 129.5 66.5) (width 0.5) (layer F.Cu) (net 12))
 (segment (start 120.5 72.6) (end 121.7 72.6) (width 0.5) (layer B.Cu) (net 12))
 (segment (start 123 71.3) (end 123 66.5) (width 0.5) (layer B.Cu) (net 12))
 (segment (start 121.7 72.6) (end 123 71.3) (width 0.5) (layer B.Cu) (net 12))
 (segment (start 120.550001 65.149999) (end 126.050001 65.149999) (width 0.5) (layer F.Cu) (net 15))
 (segment (start 120.3 65.4) (end 120.550001 65.149999) (width 0.5) (layer F.Cu) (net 15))
 (segment (start 126.050001 65.149999) (end 127.55 63.65) (width 0.5) (layer F.Cu) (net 15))
 (segment (start 127.55 63.65) (end 127.6 63.6) (width 0.5) (layer F.Cu) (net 15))
 (via (at 127.55 63.65) (size 0.8) (drill 0.4) (layers F.Cu B.Cu) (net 15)))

